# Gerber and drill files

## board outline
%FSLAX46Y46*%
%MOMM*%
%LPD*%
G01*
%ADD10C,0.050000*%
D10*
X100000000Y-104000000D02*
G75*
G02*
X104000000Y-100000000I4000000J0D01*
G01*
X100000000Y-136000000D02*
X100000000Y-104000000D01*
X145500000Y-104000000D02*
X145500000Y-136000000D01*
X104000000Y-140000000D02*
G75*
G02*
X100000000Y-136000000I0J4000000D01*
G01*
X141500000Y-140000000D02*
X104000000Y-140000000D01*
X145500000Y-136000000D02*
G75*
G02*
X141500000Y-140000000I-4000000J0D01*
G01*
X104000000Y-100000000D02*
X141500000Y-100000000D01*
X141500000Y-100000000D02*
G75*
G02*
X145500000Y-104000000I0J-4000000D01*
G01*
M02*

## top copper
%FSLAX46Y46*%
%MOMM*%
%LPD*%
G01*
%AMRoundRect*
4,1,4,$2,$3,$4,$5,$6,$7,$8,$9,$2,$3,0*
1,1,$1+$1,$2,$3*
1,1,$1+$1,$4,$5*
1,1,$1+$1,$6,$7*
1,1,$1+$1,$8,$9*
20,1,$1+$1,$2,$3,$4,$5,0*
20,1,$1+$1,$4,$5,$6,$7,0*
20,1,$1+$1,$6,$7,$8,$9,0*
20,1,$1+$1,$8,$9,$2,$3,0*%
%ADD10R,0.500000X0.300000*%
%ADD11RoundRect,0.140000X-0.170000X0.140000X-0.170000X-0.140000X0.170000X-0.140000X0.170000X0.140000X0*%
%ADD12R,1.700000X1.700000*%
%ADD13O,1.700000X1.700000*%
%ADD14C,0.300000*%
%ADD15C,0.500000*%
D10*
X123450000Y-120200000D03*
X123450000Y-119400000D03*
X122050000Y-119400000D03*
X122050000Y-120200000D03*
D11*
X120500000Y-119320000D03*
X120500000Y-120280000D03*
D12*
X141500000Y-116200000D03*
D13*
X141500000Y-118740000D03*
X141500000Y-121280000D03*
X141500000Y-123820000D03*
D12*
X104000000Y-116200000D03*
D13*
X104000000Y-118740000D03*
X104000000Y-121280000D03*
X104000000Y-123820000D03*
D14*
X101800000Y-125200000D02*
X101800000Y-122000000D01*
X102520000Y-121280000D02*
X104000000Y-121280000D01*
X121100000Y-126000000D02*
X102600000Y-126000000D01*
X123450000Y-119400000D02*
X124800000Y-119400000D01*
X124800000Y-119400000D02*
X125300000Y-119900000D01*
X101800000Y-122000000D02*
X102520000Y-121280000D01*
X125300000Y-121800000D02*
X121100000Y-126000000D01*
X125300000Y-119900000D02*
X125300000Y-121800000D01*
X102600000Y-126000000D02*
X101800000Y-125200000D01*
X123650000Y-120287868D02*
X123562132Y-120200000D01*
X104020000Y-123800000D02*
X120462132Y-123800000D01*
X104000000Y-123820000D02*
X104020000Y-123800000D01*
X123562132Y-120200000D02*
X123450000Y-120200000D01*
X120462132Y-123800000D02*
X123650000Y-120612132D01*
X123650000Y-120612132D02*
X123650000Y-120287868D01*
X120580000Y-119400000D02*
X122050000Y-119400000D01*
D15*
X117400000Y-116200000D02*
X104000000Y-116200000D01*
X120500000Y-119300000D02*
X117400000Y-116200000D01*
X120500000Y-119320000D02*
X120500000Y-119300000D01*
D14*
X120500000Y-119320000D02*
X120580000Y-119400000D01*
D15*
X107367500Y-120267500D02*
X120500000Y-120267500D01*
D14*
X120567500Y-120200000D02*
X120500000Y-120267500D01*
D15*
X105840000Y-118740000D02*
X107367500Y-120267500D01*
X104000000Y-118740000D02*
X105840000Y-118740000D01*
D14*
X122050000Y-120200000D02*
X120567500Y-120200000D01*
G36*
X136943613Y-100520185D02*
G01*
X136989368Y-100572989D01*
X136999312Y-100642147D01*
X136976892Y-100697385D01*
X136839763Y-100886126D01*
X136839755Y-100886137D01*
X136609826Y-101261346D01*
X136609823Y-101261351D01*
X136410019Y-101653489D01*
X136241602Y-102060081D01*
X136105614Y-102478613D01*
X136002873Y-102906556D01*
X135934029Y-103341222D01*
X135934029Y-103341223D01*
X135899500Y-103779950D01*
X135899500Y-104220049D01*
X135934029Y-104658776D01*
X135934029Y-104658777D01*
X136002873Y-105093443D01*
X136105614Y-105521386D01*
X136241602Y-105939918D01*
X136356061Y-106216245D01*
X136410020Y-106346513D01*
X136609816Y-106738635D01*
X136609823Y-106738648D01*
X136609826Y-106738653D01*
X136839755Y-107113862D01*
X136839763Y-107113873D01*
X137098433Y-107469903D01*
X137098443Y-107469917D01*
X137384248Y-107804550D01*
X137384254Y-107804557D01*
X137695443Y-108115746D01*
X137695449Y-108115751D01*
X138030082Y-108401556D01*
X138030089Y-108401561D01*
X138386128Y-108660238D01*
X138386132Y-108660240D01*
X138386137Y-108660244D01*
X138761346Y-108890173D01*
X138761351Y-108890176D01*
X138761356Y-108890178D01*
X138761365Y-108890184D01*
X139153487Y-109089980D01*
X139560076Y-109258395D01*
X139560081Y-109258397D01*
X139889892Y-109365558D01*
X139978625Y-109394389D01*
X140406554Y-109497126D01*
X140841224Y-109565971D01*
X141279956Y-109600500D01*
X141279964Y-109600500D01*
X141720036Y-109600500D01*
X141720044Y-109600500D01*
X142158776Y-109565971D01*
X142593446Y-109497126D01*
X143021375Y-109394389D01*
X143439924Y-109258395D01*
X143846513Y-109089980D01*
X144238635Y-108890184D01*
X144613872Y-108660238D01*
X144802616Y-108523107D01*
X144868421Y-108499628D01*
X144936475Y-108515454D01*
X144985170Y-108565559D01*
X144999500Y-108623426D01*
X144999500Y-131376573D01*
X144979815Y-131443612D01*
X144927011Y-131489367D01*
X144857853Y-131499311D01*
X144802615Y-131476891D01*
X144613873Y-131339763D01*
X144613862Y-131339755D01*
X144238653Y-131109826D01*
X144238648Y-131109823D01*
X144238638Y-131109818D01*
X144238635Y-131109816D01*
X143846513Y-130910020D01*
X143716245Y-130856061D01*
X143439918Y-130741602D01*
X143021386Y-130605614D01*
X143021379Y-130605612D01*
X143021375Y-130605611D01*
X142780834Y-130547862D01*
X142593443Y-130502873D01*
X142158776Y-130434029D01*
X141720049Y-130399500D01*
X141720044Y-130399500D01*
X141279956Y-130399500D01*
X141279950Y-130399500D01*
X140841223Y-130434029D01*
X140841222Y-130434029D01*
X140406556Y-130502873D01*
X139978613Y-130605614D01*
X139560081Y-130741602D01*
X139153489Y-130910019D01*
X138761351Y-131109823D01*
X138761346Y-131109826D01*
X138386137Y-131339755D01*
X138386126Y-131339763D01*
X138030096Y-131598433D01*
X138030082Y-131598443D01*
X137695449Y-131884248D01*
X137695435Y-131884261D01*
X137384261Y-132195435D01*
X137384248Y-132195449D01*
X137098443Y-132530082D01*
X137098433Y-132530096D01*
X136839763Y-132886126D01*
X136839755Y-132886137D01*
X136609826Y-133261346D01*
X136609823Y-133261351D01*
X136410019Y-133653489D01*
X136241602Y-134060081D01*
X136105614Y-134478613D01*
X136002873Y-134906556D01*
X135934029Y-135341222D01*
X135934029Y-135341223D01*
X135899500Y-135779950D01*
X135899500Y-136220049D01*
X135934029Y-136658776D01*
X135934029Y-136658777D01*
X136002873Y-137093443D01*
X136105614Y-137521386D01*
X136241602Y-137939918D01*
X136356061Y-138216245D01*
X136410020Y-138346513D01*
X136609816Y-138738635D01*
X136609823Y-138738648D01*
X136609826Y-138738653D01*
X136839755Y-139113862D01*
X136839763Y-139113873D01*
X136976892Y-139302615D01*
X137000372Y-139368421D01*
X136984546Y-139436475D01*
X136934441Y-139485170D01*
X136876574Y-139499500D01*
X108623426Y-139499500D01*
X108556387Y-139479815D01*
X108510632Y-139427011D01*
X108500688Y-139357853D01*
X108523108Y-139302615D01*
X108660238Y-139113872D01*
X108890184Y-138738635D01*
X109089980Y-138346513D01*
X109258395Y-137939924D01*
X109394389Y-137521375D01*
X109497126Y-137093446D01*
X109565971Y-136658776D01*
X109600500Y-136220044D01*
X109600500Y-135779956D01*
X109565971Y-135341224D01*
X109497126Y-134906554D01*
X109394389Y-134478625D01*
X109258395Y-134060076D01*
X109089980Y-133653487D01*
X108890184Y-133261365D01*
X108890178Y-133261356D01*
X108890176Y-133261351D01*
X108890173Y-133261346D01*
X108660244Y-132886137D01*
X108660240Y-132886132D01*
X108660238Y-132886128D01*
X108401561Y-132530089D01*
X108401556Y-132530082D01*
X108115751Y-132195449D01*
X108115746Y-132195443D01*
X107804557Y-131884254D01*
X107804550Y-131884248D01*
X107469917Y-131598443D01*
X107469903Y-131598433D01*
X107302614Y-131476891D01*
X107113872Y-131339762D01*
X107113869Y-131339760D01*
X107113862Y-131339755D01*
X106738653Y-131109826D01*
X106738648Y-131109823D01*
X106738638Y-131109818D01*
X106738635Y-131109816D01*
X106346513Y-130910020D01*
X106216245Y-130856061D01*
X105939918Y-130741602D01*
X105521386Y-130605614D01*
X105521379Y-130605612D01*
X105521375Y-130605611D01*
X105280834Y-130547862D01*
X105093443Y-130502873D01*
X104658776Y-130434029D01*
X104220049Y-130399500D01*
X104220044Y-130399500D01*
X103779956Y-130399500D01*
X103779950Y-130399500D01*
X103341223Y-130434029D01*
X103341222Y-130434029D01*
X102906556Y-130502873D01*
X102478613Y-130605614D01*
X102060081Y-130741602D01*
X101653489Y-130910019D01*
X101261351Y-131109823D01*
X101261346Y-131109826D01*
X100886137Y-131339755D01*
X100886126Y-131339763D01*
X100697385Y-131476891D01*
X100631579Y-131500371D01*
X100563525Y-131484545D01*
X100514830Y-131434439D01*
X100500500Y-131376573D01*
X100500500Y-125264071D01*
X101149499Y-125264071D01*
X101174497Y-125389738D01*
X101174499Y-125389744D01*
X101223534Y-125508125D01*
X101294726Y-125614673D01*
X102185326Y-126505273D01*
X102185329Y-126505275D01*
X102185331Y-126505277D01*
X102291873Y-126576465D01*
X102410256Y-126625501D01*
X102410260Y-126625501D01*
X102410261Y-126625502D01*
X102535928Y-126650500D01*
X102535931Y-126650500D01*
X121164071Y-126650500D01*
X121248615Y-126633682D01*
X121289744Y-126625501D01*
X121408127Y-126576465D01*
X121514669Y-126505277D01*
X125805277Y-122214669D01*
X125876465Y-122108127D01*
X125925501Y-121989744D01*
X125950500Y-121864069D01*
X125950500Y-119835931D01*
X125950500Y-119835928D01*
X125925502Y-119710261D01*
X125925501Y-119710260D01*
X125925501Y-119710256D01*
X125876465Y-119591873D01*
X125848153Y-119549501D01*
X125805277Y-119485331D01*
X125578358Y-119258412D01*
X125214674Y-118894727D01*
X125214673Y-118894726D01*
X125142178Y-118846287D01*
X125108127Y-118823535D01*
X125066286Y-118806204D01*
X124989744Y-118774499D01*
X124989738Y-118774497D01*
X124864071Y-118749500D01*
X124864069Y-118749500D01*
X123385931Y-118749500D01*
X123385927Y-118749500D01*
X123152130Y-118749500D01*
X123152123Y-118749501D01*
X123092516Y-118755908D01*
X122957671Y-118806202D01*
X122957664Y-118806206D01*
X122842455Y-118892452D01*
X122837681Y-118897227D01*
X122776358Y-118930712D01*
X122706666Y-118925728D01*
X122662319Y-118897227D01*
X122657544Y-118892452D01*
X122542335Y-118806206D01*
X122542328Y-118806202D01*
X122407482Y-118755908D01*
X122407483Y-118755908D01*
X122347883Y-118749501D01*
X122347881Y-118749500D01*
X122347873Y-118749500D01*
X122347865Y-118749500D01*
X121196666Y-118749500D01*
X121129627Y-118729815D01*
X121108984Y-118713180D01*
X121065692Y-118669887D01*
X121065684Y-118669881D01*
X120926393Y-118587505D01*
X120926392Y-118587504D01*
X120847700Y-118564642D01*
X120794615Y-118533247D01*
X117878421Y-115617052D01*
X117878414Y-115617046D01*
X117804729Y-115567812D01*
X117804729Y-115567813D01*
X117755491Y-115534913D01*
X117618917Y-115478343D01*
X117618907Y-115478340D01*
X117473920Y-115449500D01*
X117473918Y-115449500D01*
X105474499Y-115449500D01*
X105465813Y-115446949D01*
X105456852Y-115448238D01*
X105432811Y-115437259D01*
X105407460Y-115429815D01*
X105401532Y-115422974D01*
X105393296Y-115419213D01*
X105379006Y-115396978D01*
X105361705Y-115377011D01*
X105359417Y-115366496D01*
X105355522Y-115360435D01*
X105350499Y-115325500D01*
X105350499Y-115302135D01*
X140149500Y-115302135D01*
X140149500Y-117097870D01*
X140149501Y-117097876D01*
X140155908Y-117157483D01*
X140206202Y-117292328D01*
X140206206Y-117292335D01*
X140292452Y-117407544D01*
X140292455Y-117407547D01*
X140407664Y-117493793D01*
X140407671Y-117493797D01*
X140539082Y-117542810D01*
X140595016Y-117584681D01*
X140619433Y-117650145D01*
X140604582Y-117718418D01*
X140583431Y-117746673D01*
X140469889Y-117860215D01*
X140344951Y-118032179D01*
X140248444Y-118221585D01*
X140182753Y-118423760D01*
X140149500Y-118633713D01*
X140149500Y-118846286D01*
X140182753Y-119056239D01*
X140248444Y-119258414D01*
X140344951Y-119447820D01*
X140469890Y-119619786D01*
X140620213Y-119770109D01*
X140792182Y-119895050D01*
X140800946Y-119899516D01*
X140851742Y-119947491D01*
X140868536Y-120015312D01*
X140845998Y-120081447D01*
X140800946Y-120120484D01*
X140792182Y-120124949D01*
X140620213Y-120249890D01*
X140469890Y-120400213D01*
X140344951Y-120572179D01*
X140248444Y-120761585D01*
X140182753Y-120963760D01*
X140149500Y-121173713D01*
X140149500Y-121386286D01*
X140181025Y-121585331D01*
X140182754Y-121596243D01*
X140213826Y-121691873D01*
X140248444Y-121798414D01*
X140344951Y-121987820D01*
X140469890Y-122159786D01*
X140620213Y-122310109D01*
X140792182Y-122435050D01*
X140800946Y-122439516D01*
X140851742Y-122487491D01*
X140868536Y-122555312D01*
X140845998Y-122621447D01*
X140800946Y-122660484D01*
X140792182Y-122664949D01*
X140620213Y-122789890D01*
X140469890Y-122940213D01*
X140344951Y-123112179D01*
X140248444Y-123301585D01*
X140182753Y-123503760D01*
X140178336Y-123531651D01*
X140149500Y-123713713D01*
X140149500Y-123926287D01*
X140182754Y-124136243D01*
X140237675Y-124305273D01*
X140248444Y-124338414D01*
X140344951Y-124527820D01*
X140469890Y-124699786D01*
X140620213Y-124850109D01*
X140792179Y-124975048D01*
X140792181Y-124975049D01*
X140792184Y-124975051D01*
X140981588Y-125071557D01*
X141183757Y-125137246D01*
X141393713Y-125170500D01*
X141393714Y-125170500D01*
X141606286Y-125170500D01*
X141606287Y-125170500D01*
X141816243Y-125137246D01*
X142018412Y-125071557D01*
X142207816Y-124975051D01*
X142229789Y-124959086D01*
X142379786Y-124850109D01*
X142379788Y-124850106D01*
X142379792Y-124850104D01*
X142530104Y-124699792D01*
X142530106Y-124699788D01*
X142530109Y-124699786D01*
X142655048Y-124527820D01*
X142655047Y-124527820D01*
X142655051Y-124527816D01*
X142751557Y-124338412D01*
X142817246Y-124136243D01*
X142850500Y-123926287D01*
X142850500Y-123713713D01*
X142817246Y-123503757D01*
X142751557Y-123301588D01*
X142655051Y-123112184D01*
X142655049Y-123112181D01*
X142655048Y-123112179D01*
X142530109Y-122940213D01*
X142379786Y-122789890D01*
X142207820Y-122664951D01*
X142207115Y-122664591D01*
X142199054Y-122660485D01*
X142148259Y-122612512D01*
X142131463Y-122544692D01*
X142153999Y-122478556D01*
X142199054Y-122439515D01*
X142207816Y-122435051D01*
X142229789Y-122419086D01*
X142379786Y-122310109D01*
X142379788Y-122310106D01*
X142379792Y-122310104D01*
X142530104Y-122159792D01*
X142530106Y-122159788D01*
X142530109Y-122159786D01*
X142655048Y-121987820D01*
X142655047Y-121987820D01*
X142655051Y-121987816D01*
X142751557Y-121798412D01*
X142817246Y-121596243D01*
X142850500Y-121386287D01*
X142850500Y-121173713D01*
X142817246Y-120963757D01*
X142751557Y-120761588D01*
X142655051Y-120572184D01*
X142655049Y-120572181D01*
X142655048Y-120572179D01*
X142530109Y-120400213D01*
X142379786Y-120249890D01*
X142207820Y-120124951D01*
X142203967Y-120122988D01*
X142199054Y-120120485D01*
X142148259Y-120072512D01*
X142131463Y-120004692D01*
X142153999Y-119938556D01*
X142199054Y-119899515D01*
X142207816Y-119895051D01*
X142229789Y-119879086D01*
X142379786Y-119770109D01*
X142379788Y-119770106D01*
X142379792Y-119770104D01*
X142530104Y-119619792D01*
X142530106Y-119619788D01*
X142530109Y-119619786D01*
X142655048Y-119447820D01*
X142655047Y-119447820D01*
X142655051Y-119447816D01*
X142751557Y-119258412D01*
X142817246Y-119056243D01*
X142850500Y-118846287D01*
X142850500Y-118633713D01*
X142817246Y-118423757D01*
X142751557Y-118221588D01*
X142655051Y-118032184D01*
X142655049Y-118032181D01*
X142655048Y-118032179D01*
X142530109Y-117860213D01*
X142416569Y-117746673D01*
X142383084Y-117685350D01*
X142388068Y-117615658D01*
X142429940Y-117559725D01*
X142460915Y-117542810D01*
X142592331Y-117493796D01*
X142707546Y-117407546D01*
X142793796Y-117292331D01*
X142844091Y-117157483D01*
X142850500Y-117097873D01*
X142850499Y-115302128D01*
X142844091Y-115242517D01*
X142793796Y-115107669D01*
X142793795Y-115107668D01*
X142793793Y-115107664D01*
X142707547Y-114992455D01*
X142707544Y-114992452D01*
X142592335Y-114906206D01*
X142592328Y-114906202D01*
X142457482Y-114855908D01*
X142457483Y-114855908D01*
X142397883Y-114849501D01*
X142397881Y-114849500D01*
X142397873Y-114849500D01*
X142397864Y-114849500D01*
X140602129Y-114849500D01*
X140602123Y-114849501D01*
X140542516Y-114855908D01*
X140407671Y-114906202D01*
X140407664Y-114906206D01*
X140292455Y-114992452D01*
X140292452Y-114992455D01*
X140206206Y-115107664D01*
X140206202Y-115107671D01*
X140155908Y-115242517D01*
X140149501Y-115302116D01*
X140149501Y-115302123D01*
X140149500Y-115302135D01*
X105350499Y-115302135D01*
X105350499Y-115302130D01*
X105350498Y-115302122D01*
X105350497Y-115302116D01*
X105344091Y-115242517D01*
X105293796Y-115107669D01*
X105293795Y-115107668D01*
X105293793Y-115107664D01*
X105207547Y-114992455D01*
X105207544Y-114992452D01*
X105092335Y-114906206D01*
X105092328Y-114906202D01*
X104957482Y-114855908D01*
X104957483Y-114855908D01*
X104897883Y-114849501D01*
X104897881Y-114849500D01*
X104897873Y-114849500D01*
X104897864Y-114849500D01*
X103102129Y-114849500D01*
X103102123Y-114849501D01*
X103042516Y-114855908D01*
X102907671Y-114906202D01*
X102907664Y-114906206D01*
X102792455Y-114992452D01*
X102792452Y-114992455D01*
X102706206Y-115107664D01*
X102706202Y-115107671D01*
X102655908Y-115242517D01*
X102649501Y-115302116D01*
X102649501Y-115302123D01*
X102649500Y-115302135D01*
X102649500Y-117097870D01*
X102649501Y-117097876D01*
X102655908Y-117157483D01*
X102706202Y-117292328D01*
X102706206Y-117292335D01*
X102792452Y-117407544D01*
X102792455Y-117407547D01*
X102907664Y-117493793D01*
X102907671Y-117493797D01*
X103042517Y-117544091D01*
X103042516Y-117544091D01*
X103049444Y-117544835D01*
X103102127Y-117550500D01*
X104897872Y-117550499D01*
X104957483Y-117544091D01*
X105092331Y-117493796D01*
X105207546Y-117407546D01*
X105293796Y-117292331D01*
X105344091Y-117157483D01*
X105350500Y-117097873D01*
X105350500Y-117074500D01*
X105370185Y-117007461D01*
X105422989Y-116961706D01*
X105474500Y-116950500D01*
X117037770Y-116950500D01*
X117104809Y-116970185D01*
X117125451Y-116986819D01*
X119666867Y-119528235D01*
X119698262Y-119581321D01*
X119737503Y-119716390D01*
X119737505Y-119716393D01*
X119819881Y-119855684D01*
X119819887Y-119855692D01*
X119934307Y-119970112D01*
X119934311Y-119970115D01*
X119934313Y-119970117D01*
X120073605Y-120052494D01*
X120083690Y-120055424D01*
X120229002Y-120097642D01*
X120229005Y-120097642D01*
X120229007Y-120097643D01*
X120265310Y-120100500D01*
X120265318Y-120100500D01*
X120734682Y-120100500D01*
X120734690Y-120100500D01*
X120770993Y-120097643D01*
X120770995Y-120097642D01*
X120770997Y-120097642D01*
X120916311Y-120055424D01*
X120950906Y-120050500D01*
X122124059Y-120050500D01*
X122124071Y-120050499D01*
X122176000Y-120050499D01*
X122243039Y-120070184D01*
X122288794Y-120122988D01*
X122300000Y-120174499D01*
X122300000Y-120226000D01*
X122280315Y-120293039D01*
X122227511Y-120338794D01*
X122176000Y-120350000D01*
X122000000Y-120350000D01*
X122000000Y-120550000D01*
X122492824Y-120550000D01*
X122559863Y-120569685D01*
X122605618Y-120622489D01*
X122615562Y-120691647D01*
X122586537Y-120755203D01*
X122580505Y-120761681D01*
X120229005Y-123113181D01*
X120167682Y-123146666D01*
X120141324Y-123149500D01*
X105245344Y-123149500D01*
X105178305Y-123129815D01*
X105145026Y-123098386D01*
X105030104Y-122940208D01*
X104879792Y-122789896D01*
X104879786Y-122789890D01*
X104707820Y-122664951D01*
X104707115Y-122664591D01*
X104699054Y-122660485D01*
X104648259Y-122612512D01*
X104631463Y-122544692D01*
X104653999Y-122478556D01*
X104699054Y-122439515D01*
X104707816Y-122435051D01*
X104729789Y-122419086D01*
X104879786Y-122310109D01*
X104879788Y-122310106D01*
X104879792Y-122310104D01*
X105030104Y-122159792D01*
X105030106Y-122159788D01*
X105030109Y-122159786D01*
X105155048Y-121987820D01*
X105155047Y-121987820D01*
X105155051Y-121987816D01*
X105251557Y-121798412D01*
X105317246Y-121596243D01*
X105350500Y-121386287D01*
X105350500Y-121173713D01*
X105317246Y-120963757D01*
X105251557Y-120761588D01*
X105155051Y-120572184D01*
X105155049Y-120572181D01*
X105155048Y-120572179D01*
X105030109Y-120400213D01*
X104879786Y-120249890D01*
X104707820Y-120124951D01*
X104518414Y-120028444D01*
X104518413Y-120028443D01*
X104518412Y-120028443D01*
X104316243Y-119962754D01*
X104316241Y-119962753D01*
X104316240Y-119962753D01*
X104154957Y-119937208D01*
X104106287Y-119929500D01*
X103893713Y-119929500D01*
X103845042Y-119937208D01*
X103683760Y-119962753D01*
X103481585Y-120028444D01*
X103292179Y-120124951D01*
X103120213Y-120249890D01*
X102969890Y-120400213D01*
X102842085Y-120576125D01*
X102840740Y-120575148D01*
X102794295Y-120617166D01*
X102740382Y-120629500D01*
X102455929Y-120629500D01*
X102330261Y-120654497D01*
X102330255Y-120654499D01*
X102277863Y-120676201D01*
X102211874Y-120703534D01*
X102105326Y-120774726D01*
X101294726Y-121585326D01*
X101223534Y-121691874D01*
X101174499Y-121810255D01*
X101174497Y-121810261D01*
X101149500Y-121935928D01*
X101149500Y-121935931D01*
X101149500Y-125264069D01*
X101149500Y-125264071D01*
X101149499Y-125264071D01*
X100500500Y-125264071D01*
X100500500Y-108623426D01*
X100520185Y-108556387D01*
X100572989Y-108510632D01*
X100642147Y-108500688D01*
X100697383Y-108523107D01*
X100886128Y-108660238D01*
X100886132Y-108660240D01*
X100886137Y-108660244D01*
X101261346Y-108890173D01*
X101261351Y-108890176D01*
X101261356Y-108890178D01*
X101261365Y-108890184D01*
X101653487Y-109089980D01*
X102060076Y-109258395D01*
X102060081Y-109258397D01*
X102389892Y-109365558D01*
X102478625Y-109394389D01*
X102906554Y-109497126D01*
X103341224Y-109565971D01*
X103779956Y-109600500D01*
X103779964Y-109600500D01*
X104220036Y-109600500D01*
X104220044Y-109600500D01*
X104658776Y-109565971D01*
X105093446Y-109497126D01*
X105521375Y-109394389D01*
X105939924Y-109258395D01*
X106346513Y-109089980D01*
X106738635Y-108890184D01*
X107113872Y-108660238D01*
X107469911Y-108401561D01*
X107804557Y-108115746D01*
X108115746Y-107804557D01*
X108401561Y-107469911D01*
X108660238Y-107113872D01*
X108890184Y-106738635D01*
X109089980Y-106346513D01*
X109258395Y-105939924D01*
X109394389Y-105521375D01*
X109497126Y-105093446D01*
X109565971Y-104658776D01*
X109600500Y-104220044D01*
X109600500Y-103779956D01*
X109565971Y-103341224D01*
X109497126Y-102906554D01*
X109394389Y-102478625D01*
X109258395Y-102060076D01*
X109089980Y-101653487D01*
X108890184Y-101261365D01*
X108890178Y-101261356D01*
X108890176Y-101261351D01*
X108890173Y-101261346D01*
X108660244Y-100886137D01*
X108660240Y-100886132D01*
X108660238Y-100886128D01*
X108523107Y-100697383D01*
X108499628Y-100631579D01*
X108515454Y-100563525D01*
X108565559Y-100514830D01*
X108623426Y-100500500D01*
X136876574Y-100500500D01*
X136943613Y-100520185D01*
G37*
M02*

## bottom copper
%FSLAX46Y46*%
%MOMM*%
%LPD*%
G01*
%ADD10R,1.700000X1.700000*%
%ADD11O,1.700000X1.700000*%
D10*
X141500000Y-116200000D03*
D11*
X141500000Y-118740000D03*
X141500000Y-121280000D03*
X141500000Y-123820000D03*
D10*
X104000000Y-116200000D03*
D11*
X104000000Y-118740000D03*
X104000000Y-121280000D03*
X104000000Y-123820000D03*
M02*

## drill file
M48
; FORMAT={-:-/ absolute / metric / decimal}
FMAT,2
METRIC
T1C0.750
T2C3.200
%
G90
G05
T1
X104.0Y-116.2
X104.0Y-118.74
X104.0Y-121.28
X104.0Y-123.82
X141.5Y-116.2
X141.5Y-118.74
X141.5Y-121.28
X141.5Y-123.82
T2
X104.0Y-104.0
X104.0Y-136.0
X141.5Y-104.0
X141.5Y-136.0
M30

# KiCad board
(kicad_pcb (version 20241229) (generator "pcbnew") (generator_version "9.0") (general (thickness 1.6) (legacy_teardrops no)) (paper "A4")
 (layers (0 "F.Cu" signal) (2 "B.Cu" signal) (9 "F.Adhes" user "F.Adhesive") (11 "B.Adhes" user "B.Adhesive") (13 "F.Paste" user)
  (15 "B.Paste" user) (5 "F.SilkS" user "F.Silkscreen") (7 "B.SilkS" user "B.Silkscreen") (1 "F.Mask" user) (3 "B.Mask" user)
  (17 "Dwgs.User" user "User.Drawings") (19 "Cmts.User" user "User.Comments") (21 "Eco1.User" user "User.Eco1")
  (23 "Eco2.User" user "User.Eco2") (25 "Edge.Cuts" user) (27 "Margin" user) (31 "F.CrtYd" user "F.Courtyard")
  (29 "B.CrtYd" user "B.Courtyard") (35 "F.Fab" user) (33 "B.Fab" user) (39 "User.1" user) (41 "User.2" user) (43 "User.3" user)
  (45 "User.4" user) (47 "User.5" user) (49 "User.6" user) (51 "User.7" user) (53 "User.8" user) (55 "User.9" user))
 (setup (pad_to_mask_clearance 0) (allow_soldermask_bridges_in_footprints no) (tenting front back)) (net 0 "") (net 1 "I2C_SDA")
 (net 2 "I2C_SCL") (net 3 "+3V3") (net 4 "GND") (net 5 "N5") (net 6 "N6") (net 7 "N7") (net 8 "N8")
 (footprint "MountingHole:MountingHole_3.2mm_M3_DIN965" (layer "F.Cu") (at 141.5 104)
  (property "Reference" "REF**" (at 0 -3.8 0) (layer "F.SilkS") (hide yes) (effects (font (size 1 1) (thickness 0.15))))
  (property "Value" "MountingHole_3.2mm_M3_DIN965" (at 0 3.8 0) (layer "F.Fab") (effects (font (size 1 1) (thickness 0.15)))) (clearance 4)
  (pad "" np_thru_hole circle (at 0 0) (size 3.2 3.2) (drill 3.2) (layers "*.Cu" "*.Mask")))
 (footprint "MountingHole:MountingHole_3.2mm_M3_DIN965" (layer "F.Cu") (at 141.5 136)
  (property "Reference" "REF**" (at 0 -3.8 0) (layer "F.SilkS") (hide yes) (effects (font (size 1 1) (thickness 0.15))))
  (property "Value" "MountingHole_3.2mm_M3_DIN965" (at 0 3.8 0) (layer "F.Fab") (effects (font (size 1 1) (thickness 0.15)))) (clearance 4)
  (pad "" np_thru_hole circle (at 0 0) (size 3.2 3.2) (drill 3.2) (layers "*.Cu" "*.Mask")))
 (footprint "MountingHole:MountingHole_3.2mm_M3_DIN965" (layer "F.Cu") (at 104 136)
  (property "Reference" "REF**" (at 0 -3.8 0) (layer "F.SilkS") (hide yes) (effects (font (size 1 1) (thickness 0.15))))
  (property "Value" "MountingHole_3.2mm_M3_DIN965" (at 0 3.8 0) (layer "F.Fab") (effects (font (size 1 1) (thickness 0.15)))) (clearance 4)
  (pad "" np_thru_hole circle (at 0 0) (size 3.2 3.2) (drill 3.2) (layers "*.Cu" "*.Mask")))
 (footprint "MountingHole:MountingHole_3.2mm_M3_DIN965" (layer "F.Cu") (at 104 104)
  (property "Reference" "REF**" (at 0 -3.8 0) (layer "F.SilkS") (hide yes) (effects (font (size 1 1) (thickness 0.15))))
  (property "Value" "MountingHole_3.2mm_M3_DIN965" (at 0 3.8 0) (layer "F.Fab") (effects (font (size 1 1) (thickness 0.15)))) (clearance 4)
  (pad "" np_thru_hole circle (at 0 0) (size 3.2 3.2) (drill 3.2) (layers "*.Cu" "*.Mask")))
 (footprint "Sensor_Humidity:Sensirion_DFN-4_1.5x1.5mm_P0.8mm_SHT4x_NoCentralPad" (layer "F.Cu") (at 122.75 119.8 180)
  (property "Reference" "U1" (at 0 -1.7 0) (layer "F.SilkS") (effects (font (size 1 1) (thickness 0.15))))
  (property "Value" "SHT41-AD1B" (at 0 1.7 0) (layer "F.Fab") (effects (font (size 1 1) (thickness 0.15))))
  (pad "1" smd rect (at -0.7 -0.4 180) (size 0.5 0.3) (layers "F.Cu" "F.Mask" "F.Paste") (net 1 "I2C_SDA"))
  (pad "2" smd rect (at -0.7 0.4 180) (size 0.5 0.3) (layers "F.Cu" "F.Mask" "F.Paste") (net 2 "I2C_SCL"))
  (pad "3" smd rect (at 0.7 0.4 180) (size 0.5 0.3) (layers "F.Cu" "F.Mask" "F.Paste") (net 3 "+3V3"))
  (pad "4" smd rect (at 0.7 -0.4 180) (size 0.5 0.3) (layers "F.Cu" "F.Mask" "F.Paste") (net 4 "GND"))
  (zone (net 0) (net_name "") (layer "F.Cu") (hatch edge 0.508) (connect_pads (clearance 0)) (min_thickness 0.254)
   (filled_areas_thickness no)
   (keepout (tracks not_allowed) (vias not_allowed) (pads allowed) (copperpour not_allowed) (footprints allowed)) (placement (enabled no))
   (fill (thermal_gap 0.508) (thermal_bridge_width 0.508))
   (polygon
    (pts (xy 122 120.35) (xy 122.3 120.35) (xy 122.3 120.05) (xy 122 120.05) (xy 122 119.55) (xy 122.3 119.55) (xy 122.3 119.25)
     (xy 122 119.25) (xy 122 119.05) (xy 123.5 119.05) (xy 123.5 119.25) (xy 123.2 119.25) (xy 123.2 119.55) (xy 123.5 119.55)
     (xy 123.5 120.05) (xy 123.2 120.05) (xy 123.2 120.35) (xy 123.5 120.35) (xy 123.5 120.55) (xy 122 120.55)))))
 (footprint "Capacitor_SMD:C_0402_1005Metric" (layer "F.Cu") (at 120.5 119.8 -90)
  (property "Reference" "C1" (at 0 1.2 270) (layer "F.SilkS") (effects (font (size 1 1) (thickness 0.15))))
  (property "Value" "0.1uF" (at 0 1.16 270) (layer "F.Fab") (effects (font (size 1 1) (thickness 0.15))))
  (pad "1" smd roundrect (at -0.48 0 270) (size 0.56 0.62) (layers "F.Cu" "F.Mask" "F.Paste") (roundrect_rratio 0.25) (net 3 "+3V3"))
  (pad "2" smd roundrect (at 0.48 0 270) (size 0.56 0.62) (layers "F.Cu" "F.Mask" "F.Paste") (roundrect_rratio 0.25) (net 4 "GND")))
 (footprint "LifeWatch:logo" (layer "F.Cu") (at 133.1 119.9)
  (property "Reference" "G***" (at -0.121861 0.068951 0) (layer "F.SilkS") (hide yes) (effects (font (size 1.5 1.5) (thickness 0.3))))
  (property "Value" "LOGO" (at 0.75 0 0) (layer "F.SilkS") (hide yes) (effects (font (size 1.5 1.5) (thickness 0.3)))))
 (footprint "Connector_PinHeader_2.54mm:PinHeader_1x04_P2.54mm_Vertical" (layer "B.Cu") (at 141.5 116.2 180)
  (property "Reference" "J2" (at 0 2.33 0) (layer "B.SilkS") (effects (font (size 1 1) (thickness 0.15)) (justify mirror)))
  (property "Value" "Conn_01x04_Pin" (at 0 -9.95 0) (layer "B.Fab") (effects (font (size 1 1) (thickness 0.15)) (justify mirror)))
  (pad "1" thru_hole rect (at 0 0 180) (size 1.7 1.7) (drill 0.75) (layers "*.Cu" "*.Mask") (remove_unused_layers no) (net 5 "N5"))
  (pad "2" thru_hole oval (at 0 -2.54 180) (size 1.7 1.7) (drill 0.75) (layers "*.Cu" "*.Mask") (remove_unused_layers no) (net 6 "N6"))
  (pad "3" thru_hole oval (at 0 -5.08 180) (size 1.7 1.7) (drill 0.75) (layers "*.Cu" "*.Mask") (remove_unused_layers no) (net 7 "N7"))
  (pad "4" thru_hole oval (at 0 -7.62 180) (size 1.7 1.7) (drill 0.75) (layers "*.Cu" "*.Mask") (remove_unused_layers no) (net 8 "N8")))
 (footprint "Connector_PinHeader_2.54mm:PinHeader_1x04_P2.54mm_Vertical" (layer "B.Cu") (at 104 116.2 180)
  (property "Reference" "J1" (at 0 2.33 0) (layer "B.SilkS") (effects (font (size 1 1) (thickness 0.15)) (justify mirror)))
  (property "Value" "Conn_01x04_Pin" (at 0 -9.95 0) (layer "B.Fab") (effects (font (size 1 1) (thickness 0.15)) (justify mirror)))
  (pad "1" thru_hole rect (at 0 0 180) (size 1.7 1.7) (drill 0.75) (layers "*.Cu" "*.Mask") (remove_unused_layers no) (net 3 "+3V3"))
  (pad "2" thru_hole oval (at 0 -2.54 180) (size 1.7 1.7) (drill 0.75) (layers "*.Cu" "*.Mask") (remove_unused_layers no) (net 4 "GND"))
  (pad "3" thru_hole oval (at 0 -5.08 180) (size 1.7 1.7) (drill 0.75) (layers "*.Cu" "*.Mask") (remove_unused_layers no) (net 2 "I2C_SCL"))
  (pad "4" thru_hole oval (at 0 -7.62 180) (size 1.7 1.7) (drill 0.75) (layers "*.Cu" "*.Mask") (remove_unused_layers no) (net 1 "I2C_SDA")))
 (gr_arc (start 100 104) (mid 101.171573 101.171573) (end 104 100) (stroke (width 0.05) (type default)) (layer "Edge.Cuts"))
 (gr_line (start 100 136) (end 100 104) (stroke (width 0.05) (type default)) (layer "Edge.Cuts"))
 (gr_line (start 145.5 104) (end 145.5 136) (stroke (width 0.05) (type default)) (layer "Edge.Cuts"))
 (gr_arc (start 104 140) (mid 101.171573 138.828427) (end 100 136) (stroke (width 0.05) (type default)) (layer "Edge.Cuts"))
 (gr_line (start 141.5 140) (end 104 140) (stroke (width 0.05) (type default)) (layer "Edge.Cuts"))
 (gr_arc (start 145.5 136) (mid 144.328427 138.828427) (end 141.5 140) (stroke (width 0.05) (type default)) (layer "Edge.Cuts"))
 (gr_line (start 104 100) (end 141.5 100) (stroke (width 0.05) (type default)) (layer "Edge.Cuts"))
 (gr_arc (start 141.5 100) (mid 144.328427 101.171573) (end 145.5 104) (stroke (width 0.05) (type default)) (layer "Edge.Cuts"))
 (segment (start 101.8 125.2) (end 101.8 122) (width 0.3) (layer "F.Cu") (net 2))
 (segment (start 102.52 121.28) (end 104 121.28) (width 0.3) (layer "F.Cu") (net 2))
 (segment (start 121.1 126) (end 102.6 126) (width 0.3) (layer "F.Cu") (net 2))
 (segment (start 123.45 119.4) (end 124.8 119.4) (width 0.3) (layer "F.Cu") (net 2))
 (segment (start 124.8 119.4) (end 125.3 119.9) (width 0.3) (layer "F.Cu") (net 2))
 (segment (start 101.8 122) (end 102.52 121.28) (width 0.3) (layer "F.Cu") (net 2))
 (segment (start 125.3 121.8) (end 121.1 126) (width 0.3) (layer "F.Cu") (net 2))
 (segment (start 125.3 119.9) (end 125.3 121.8) (width 0.3) (layer "F.Cu") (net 2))
 (segment (start 102.6 126) (end 101.8 125.2) (width 0.3) (layer "F.Cu") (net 2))
 (segment (start 123.65 120.287868) (end 123.562132 120.2) (width 0.3) (layer "F.Cu") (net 1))
 (segment (start 104.02 123.8) (end 120.462132 123.8) (width 0.3) (layer "F.Cu") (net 1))
 (segment (start 104 123.82) (end 104.02 123.8) (width 0.3) (layer "F.Cu") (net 1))
 (segment (start 123.562132 120.2) (end 123.45 120.2) (width 0.3) (layer "F.Cu") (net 1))
 (segment (start 120.462132 123.8) (end 123.65 120.612132) (width 0.3) (layer "F.Cu") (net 1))
 (segment (start 123.65 120.612132) (end 123.65 120.287868) (width 0.3) (layer "F.Cu") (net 1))
 (segment (start 120.58 119.4) (end 122.05 119.4) (width 0.3) (layer "F.Cu") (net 3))
 (segment (start 117.4 116.2) (end 104 116.2) (width 0.5) (layer "F.Cu") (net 3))
 (segment (start 120.5 119.3) (end 117.4 116.2) (width 0.5) (layer "F.Cu") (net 3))
 (segment (start 120.5 119.32) (end 120.5 119.3) (width 0.5) (layer "F.Cu") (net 3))
 (segment (start 120.5 119.32) (end 120.58 119.4) (width 0.3) (layer "F.Cu") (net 3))
 (segment (start 107.3675 120.2675) (end 120.5 120.2675) (width 0.5) (layer "F.Cu") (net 4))
 (segment (start 120.5675 120.2) (end 120.5 120.2675) (width 0.3) (layer "F.Cu") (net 4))
 (segment (start 105.84 118.74) (end 107.3675 120.2675) (width 0.5) (layer "F.Cu") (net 4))
 (segment (start 104 118.74) (end 105.84 118.74) (width 0.5) (layer "F.Cu") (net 4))
 (segment (start 122.05 120.2) (end 120.5675 120.2) (width 0.3) (layer "F.Cu") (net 4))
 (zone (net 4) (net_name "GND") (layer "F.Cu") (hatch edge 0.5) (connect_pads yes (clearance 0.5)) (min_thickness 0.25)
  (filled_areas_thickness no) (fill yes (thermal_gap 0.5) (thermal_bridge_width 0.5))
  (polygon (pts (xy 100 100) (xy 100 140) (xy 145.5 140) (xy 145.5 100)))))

